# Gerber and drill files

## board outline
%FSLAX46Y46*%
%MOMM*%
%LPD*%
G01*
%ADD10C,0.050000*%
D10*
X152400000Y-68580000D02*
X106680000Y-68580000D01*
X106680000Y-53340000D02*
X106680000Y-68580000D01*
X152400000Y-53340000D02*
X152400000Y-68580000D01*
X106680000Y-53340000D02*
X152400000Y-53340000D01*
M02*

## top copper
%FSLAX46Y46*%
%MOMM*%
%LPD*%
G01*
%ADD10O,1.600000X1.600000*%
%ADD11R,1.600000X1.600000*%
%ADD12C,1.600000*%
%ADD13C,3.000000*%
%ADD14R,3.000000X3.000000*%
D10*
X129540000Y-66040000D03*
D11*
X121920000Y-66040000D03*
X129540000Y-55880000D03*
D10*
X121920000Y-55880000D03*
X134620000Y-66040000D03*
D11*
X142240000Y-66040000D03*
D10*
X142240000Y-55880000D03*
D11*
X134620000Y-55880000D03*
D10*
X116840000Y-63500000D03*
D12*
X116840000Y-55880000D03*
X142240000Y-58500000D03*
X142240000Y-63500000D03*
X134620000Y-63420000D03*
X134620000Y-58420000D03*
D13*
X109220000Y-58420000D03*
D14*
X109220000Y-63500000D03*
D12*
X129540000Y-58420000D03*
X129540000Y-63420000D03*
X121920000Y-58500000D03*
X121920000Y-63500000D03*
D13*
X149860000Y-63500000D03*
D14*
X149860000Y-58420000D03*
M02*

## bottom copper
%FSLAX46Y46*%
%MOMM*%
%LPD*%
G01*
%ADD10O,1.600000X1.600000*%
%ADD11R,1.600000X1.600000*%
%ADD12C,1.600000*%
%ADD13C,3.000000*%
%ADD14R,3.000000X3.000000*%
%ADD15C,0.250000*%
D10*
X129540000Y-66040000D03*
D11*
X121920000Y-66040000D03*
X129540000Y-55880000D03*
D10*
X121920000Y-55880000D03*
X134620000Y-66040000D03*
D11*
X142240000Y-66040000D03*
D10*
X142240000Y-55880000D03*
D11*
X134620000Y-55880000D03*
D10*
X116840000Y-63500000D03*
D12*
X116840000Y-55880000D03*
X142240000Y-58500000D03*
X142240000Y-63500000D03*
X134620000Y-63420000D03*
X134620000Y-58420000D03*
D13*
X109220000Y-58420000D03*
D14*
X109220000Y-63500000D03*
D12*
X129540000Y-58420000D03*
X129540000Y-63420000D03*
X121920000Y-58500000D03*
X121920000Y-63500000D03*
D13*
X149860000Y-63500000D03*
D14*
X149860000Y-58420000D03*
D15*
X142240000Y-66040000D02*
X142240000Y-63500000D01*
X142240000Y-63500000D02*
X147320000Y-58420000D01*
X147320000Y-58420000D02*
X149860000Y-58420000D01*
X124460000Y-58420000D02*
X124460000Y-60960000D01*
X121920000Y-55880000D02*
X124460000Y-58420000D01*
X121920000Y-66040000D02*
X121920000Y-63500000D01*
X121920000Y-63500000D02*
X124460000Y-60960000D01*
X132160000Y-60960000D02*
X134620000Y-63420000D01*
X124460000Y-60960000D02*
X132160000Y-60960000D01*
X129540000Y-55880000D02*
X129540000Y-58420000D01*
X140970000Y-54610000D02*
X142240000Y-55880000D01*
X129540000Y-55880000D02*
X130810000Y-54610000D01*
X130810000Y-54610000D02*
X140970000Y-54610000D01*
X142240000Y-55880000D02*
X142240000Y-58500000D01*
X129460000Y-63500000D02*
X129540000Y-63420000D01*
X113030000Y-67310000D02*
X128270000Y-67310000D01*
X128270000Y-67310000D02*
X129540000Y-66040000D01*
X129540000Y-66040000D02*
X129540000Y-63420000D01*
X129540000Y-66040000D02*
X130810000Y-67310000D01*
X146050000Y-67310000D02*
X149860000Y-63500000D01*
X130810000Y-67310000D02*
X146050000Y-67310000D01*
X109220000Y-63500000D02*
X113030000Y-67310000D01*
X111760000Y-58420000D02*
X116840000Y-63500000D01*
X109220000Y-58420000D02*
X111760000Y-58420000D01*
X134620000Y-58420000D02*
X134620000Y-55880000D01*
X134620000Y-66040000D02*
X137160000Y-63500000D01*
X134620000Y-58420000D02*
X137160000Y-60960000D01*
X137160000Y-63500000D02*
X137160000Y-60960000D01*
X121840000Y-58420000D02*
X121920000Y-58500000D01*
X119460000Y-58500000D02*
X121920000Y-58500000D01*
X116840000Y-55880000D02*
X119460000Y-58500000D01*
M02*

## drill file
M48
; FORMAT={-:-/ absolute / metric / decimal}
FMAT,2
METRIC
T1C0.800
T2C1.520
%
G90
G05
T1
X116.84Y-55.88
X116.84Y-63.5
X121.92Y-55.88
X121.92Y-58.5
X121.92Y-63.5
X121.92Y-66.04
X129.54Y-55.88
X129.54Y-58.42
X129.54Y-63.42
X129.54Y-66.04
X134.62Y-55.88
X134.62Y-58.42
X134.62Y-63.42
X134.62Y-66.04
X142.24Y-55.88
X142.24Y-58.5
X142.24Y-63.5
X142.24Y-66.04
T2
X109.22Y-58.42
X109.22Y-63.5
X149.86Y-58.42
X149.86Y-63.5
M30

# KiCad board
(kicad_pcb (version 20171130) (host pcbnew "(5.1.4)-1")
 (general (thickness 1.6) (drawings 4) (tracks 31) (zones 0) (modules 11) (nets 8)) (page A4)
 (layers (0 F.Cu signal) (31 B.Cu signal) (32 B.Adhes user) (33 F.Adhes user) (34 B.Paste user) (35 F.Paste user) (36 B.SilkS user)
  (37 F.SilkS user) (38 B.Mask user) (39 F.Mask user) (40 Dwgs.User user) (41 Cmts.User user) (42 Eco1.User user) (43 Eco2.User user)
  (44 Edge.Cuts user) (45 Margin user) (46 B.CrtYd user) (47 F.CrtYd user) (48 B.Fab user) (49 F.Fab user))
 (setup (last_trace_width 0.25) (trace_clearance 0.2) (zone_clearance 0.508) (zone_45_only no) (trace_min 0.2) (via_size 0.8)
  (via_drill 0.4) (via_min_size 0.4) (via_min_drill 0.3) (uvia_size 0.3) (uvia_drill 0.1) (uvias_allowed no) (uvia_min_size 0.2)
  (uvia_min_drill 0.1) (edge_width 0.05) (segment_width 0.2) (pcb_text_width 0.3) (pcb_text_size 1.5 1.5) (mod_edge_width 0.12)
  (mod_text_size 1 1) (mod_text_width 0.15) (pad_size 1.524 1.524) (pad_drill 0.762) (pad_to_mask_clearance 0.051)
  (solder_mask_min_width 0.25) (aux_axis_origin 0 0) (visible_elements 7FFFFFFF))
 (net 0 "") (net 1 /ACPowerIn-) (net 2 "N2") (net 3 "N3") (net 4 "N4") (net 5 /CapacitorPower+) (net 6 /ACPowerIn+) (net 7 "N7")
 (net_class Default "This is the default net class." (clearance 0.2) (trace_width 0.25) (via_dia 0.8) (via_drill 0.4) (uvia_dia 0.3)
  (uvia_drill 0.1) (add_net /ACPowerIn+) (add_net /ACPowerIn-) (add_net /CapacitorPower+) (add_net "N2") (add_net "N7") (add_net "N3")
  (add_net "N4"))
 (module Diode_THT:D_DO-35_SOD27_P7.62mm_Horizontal (layer F.Cu) (at 121.92 66.04)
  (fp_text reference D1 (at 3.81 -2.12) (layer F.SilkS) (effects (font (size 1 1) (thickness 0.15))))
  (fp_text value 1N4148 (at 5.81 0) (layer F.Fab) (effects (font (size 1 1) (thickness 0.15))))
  (pad 2 thru_hole oval (at 7.62 0) (size 1.6 1.6) (drill 0.8) (layers *.Cu *.Mask) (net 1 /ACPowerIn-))
  (pad 1 thru_hole rect (at 0 0) (size 1.6 1.6) (drill 0.8) (layers *.Cu *.Mask) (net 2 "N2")))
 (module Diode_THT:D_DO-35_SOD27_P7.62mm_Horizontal (layer F.Cu) (at 129.54 55.88 180)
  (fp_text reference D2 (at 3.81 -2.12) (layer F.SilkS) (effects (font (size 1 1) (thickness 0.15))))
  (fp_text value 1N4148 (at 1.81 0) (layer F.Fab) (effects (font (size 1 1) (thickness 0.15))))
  (pad 1 thru_hole rect (at 0 0 180) (size 1.6 1.6) (drill 0.8) (layers *.Cu *.Mask) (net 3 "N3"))
  (pad 2 thru_hole oval (at 7.62 0 180) (size 1.6 1.6) (drill 0.8) (layers *.Cu *.Mask) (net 2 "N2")))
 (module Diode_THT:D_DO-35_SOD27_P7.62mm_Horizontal (layer F.Cu) (at 142.24 66.04 180)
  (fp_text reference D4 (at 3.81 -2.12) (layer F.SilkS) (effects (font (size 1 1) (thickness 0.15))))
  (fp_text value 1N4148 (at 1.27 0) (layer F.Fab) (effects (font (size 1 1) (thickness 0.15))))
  (pad 2 thru_hole oval (at 7.62 0 180) (size 1.6 1.6) (drill 0.8) (layers *.Cu *.Mask) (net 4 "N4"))
  (pad 1 thru_hole rect (at 0 0 180) (size 1.6 1.6) (drill 0.8) (layers *.Cu *.Mask) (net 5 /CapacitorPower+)))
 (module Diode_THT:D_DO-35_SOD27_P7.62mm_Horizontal (layer F.Cu) (at 134.62 55.88)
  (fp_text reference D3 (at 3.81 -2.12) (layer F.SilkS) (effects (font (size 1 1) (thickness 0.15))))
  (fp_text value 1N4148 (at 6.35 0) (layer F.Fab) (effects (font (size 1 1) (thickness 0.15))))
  (pad 2 thru_hole oval (at 7.62 0) (size 1.6 1.6) (drill 0.8) (layers *.Cu *.Mask) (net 3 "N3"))
  (pad 1 thru_hole rect (at 0 0) (size 1.6 1.6) (drill 0.8) (layers *.Cu *.Mask) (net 4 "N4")))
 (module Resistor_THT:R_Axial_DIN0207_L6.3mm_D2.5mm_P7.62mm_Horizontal (layer F.Cu) (at 116.84 55.88 270)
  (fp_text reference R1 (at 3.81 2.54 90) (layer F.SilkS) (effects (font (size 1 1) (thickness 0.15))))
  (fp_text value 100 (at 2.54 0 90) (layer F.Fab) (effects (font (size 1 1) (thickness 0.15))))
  (pad 2 thru_hole oval (at 7.62 0 270) (size 1.6 1.6) (drill 0.8) (layers *.Cu *.Mask) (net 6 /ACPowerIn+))
  (pad 1 thru_hole circle (at 0 0 270) (size 1.6 1.6) (drill 0.8) (layers *.Cu *.Mask) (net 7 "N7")))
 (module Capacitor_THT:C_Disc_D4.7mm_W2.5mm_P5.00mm (layer F.Cu) (at 142.24 63.5 90)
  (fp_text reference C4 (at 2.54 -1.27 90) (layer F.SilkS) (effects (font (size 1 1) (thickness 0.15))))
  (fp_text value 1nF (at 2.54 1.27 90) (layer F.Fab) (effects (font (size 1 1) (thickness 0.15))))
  (pad 2 thru_hole circle (at 5 0 90) (size 1.6 1.6) (drill 0.8) (layers *.Cu *.Mask) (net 3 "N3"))
  (pad 1 thru_hole circle (at 0 0 90) (size 1.6 1.6) (drill 0.8) (layers *.Cu *.Mask) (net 5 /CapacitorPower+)))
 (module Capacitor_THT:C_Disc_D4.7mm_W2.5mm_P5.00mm (layer F.Cu) (at 134.62 58.42 270)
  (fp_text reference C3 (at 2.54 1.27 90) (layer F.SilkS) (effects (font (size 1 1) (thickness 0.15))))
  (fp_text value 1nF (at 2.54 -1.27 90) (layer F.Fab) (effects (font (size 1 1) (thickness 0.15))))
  (pad 2 thru_hole circle (at 5 0 270) (size 1.6 1.6) (drill 0.8) (layers *.Cu *.Mask) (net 2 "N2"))
  (pad 1 thru_hole circle (at 0 0 270) (size 1.6 1.6) (drill 0.8) (layers *.Cu *.Mask) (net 4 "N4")))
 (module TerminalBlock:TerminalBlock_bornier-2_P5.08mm (layer F.Cu) (at 109.22 63.5 90)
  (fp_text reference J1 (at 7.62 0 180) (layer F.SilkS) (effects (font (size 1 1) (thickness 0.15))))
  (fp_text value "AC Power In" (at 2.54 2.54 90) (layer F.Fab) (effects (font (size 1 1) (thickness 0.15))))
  (pad 2 thru_hole circle (at 5.08 0 90) (size 3 3) (drill 1.52) (layers *.Cu *.Mask) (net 6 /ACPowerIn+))
  (pad 1 thru_hole rect (at 0 0 90) (size 3 3) (drill 1.52) (layers *.Cu *.Mask) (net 1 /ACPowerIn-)))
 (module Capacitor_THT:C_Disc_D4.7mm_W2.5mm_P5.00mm (layer F.Cu) (at 129.54 58.42 270)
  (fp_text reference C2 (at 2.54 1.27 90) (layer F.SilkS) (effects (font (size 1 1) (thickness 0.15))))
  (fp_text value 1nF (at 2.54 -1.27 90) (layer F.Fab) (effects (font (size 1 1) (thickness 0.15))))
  (pad 1 thru_hole circle (at 0 0 270) (size 1.6 1.6) (drill 0.8) (layers *.Cu *.Mask) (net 3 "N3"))
  (pad 2 thru_hole circle (at 5 0 270) (size 1.6 1.6) (drill 0.8) (layers *.Cu *.Mask) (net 1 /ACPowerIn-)))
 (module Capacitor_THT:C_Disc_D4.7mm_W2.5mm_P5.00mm (layer F.Cu) (at 121.92 63.5 90)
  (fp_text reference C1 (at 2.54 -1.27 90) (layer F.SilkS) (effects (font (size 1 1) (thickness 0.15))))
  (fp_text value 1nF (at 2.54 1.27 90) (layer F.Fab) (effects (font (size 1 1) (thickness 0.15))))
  (pad 2 thru_hole circle (at 5 0 90) (size 1.6 1.6) (drill 0.8) (layers *.Cu *.Mask) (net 7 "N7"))
  (pad 1 thru_hole circle (at 0 0 90) (size 1.6 1.6) (drill 0.8) (layers *.Cu *.Mask) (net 2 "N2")))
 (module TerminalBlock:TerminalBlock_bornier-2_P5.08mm (layer F.Cu) (at 149.86 58.42 270)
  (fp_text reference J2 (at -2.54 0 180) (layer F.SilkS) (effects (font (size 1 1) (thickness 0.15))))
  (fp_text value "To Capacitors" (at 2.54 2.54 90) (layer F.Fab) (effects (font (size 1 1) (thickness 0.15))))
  (pad 2 thru_hole circle (at 5.08 0 270) (size 3 3) (drill 1.52) (layers *.Cu *.Mask) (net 1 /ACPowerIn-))
  (pad 1 thru_hole rect (at 0 0 270) (size 3 3) (drill 1.52) (layers *.Cu *.Mask) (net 5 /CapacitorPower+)))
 (gr_line (start 152.4 68.58) (end 106.68 68.58) (layer Edge.Cuts) (width 0.05))
 (gr_line (start 106.68 53.34) (end 106.68 68.58) (layer Edge.Cuts) (width 0.05))
 (gr_line (start 152.4 53.34) (end 152.4 68.58) (layer Edge.Cuts) (width 0.05))
 (gr_line (start 106.68 53.34) (end 152.4 53.34) (layer Edge.Cuts) (width 0.05))
 (segment (start 142.24 66.04) (end 142.24 63.5) (width 0.25) (layer B.Cu) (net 5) (status 30))
 (segment (start 142.24 63.5) (end 147.32 58.42) (width 0.25) (layer B.Cu) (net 5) (status 10))
 (segment (start 147.32 58.42) (end 149.86 58.42) (width 0.25) (layer B.Cu) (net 5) (status 20))
 (segment (start 124.46 58.42) (end 124.46 60.96) (width 0.25) (layer B.Cu) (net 2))
 (segment (start 121.92 55.88) (end 124.46 58.42) (width 0.25) (layer B.Cu) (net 2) (status 10))
 (segment (start 121.92 66.04) (end 121.92 63.5) (width 0.25) (layer B.Cu) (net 2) (status 30))
 (segment (start 121.92 63.5) (end 124.46 60.96) (width 0.25) (layer B.Cu) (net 2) (status 10))
 (segment (start 132.16 60.96) (end 134.62 63.42) (width 0.25) (layer B.Cu) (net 2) (status 20))
 (segment (start 124.46 60.96) (end 132.16 60.96) (width 0.25) (layer B.Cu) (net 2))
 (segment (start 129.54 55.88) (end 129.54 58.42) (width 0.25) (layer B.Cu) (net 3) (status 30))
 (segment (start 140.97 54.61) (end 142.24 55.88) (width 0.25) (layer B.Cu) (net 3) (status 20))
 (segment (start 129.54 55.88) (end 130.81 54.61) (width 0.25) (layer B.Cu) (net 3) (status 10))
 (segment (start 130.81 54.61) (end 140.97 54.61) (width 0.25) (layer B.Cu) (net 3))
 (segment (start 142.24 55.88) (end 142.24 58.5) (width 0.25) (layer B.Cu) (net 3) (status 30))
 (segment (start 129.46 63.5) (end 129.54 63.42) (width 0.25) (layer B.Cu) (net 1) (status 30))
 (segment (start 113.03 67.31) (end 128.27 67.31) (width 0.25) (layer B.Cu) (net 1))
 (segment (start 128.27 67.31) (end 129.54 66.04) (width 0.25) (layer B.Cu) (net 1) (status 20))
 (segment (start 129.54 66.04) (end 129.54 63.42) (width 0.25) (layer B.Cu) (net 1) (status 30))
 (segment (start 129.54 66.04) (end 130.81 67.31) (width 0.25) (layer B.Cu) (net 1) (status 10))
 (segment (start 146.05 67.31) (end 149.86 63.5) (width 0.25) (layer B.Cu) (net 1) (status 20))
 (segment (start 130.81 67.31) (end 146.05 67.31) (width 0.25) (layer B.Cu) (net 1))
 (segment (start 109.22 63.5) (end 113.03 67.31) (width 0.25) (layer B.Cu) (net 1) (status 10))
 (segment (start 111.76 58.42) (end 116.84 63.5) (width 0.25) (layer B.Cu) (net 6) (status 20))
 (segment (start 109.22 58.42) (end 111.76 58.42) (width 0.25) (layer B.Cu) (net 6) (status 10))
 (segment (start 134.62 58.42) (end 134.62 55.88) (width 0.25) (layer B.Cu) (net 4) (status 30))
 (segment (start 134.62 66.04) (end 137.16 63.5) (width 0.25) (layer B.Cu) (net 4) (status 10))
 (segment (start 134.62 58.42) (end 137.16 60.96) (width 0.25) (layer B.Cu) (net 4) (status 10))
 (segment (start 137.16 63.5) (end 137.16 60.96) (width 0.25) (layer B.Cu) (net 4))
 (segment (start 121.84 58.42) (end 121.92 58.5) (width 0.25) (layer B.Cu) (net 7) (status 30))
 (segment (start 119.46 58.5) (end 121.92 58.5) (width 0.25) (layer B.Cu) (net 7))
 (segment (start 116.84 55.88) (end 119.46 58.5) (width 0.25) (layer B.Cu) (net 7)))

